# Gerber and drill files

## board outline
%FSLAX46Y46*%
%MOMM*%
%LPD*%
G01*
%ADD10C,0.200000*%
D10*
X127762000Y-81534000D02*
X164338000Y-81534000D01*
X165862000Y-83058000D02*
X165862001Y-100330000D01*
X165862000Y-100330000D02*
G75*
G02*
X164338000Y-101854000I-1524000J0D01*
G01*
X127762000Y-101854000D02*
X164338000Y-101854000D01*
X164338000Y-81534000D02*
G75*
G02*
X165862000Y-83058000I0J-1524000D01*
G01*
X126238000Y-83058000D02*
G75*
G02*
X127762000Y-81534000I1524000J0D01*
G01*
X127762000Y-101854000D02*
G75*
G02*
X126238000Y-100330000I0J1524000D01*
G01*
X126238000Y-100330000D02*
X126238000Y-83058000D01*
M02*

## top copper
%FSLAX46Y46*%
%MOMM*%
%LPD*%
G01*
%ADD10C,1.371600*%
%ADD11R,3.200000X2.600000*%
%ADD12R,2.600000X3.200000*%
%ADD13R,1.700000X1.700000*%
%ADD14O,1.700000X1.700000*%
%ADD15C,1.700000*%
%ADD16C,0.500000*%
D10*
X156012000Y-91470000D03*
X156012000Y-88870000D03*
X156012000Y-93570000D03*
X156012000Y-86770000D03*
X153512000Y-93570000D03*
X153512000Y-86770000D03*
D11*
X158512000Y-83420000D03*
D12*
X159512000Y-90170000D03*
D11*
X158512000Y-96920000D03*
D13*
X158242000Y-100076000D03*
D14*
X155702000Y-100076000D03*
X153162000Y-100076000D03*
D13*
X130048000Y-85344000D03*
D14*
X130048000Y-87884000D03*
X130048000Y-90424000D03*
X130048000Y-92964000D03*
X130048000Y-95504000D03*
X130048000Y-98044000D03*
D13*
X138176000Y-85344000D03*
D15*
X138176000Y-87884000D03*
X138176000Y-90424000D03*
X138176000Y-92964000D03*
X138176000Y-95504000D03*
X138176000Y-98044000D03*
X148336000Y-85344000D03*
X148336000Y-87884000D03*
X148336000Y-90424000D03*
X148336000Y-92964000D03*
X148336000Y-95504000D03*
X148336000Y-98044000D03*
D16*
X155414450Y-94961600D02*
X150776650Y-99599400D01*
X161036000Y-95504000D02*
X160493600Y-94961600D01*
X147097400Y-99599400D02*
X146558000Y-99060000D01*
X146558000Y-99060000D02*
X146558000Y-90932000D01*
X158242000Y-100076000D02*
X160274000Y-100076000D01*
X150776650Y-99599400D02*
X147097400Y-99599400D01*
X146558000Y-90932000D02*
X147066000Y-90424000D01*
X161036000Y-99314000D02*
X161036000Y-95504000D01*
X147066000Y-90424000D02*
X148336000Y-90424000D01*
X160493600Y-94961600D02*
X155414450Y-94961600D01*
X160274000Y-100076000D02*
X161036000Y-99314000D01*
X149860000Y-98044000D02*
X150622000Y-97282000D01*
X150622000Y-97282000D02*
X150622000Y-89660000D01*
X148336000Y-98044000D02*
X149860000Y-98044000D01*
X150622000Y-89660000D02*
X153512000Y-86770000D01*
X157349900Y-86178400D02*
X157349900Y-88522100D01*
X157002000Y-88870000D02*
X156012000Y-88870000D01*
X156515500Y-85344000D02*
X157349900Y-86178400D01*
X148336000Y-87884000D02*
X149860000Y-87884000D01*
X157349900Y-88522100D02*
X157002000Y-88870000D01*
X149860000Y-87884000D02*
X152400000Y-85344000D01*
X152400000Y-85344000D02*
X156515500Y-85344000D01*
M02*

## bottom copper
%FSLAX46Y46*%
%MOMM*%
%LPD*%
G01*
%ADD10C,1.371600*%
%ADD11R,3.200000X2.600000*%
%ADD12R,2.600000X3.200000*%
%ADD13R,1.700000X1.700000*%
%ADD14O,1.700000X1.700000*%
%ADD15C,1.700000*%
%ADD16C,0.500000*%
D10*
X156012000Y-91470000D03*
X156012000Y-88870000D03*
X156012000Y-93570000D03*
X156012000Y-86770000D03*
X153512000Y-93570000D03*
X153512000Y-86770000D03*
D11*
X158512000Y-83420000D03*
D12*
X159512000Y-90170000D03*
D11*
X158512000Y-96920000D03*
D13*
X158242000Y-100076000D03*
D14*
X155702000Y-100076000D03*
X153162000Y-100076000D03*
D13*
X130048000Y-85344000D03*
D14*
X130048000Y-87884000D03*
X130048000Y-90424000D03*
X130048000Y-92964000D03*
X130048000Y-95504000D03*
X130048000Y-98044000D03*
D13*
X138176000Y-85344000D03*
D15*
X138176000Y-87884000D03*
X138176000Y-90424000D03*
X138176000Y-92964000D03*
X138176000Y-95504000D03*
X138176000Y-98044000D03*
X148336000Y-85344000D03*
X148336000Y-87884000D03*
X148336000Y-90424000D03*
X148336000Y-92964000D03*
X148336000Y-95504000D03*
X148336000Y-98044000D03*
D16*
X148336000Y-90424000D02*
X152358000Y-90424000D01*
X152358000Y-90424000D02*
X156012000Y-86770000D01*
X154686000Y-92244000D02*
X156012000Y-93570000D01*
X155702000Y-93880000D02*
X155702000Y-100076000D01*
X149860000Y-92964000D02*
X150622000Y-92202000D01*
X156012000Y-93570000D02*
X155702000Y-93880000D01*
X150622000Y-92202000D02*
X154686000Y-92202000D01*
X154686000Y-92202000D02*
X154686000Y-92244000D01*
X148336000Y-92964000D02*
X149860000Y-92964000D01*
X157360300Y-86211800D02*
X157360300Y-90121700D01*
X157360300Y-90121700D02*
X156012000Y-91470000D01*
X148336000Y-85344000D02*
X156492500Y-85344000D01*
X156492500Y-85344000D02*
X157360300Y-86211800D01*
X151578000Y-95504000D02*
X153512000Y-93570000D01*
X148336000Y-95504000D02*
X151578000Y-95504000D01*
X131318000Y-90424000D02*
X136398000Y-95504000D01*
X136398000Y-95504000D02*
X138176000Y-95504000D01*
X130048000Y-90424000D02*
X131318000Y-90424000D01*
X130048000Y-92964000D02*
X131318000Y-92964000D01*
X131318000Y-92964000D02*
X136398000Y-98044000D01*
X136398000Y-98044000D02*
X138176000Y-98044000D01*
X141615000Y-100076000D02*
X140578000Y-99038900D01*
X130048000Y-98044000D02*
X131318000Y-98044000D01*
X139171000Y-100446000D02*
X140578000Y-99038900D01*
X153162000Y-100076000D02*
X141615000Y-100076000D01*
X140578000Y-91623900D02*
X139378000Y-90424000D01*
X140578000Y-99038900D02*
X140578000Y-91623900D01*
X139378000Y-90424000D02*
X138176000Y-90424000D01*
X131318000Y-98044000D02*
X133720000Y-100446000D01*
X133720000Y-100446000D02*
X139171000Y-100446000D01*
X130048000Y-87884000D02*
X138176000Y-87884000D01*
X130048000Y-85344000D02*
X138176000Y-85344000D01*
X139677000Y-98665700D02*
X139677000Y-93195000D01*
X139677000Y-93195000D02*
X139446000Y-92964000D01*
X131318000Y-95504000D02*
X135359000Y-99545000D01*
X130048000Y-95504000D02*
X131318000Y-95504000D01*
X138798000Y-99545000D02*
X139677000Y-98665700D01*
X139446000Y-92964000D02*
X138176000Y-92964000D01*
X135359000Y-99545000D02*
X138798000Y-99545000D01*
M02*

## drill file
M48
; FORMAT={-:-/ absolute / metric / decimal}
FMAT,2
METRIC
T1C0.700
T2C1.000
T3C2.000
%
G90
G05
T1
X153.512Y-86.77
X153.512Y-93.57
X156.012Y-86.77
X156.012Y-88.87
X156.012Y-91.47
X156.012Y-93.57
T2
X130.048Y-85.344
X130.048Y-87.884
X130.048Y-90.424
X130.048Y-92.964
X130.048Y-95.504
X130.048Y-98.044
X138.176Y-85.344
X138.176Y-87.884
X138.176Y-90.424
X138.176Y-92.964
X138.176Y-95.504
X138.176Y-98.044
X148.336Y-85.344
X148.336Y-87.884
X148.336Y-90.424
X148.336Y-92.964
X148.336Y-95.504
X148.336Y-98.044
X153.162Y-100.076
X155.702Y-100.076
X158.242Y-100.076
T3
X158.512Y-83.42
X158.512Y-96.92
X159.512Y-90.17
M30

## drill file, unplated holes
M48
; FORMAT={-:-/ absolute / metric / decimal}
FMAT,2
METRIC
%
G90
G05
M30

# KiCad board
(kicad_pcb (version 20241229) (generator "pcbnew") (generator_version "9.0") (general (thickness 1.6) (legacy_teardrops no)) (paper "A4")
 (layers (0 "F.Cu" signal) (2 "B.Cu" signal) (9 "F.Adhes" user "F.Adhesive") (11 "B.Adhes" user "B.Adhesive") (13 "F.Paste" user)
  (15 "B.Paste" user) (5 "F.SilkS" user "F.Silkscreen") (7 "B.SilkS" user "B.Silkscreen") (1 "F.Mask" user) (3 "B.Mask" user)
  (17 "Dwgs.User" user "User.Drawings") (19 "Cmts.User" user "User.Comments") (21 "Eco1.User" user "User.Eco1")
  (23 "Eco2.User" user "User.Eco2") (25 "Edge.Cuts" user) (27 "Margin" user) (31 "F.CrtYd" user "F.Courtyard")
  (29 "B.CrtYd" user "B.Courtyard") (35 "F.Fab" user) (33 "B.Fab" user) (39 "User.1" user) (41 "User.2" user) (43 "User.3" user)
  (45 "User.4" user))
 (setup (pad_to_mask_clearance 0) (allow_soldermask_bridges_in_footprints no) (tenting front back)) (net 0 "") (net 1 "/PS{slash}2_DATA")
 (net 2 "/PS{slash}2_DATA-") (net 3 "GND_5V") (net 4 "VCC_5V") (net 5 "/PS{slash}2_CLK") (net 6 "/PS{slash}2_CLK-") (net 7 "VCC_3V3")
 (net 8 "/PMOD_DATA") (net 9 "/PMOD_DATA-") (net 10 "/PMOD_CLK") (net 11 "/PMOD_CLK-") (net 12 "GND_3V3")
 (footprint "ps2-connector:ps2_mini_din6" (layer "F.Cu") (at 158.512 90.17 -90)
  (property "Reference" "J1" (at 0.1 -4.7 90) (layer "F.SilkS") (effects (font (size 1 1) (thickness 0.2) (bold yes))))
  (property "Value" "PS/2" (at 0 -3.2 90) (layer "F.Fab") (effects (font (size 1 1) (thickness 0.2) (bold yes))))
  (pad "1" thru_hole circle (at 1.3 2.5 90) (size 1.3716 1.3716) (drill 0.7) (layers "*.Cu" "*.Mask") (remove_unused_layers no)
   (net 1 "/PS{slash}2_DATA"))
  (pad "2" thru_hole circle (at -1.3 2.5 90) (size 1.3716 1.3716) (drill 0.7) (layers "*.Cu" "*.Mask") (remove_unused_layers no)
   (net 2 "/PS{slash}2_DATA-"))
  (pad "3" thru_hole circle (at 3.4 2.5 90) (size 1.3716 1.3716) (drill 0.7) (layers "*.Cu" "*.Mask") (remove_unused_layers no)
   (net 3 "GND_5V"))
  (pad "4" thru_hole circle (at -3.4 2.5 90) (size 1.3716 1.3716) (drill 0.7) (layers "*.Cu" "*.Mask") (remove_unused_layers no)
   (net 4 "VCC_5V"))
  (pad "5" thru_hole circle (at 3.4 5 90) (size 1.3716 1.3716) (drill 0.7) (layers "*.Cu" "*.Mask") (remove_unused_layers no)
   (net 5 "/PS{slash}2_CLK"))
  (pad "6" thru_hole circle (at -3.4 5 90) (size 1.3716 1.3716) (drill 0.7) (layers "*.Cu" "*.Mask") (remove_unused_layers no)
   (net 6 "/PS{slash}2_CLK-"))
  (pad "GND" thru_hole rect (at -6.75 0 90) (size 2.6 3.2) (drill 2) (layers "*.Cu" "*.Mask") (remove_unused_layers no)
   (thermal_bridge_angle 45))
  (pad "GND" thru_hole rect (at 0 -1 90) (size 3.2 2.6) (drill 2) (layers "*.Cu" "*.Mask") (remove_unused_layers no)
   (thermal_bridge_angle 45))
  (pad "GND" thru_hole rect (at 6.75 0 90) (size 2.6 3.2) (drill 2) (layers "*.Cu" "*.Mask") (remove_unused_layers no)
   (thermal_bridge_angle 45)))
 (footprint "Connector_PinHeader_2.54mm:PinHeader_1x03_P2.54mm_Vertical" (layer "F.Cu") (at 158.242 100.076 -90)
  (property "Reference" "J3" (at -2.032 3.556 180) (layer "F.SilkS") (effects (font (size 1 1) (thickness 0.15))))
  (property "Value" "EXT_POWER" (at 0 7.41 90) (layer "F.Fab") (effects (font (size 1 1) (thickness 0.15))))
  (pad "1" thru_hole rect (at 0 0 270) (size 1.7 1.7) (drill 1) (layers "*.Cu" "*.Mask") (remove_unused_layers no) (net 4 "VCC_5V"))
  (pad "2" thru_hole oval (at 0 2.54 270) (size 1.7 1.7) (drill 1) (layers "*.Cu" "*.Mask") (remove_unused_layers no) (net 3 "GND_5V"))
  (pad "3" thru_hole oval (at 0 5.08 270) (size 1.7 1.7) (drill 1) (layers "*.Cu" "*.Mask") (remove_unused_layers no) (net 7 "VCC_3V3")))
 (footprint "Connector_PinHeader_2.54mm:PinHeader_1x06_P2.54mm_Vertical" (layer "F.Cu") (at 130.048 85.344)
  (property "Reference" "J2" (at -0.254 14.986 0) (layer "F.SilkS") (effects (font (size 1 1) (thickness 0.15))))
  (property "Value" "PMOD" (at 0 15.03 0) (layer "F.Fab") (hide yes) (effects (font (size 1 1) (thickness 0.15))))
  (pad "1" thru_hole rect (at 0 0) (size 1.7 1.7) (drill 1) (layers "*.Cu" "*.Mask") (remove_unused_layers no) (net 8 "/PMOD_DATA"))
  (pad "2" thru_hole oval (at 0 2.54) (size 1.7 1.7) (drill 1) (layers "*.Cu" "*.Mask") (remove_unused_layers no) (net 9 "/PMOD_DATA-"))
  (pad "3" thru_hole oval (at 0 5.08) (size 1.7 1.7) (drill 1) (layers "*.Cu" "*.Mask") (remove_unused_layers no) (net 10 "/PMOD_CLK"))
  (pad "4" thru_hole oval (at 0 7.62) (size 1.7 1.7) (drill 1) (layers "*.Cu" "*.Mask") (remove_unused_layers no) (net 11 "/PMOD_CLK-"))
  (pad "5" thru_hole oval (at 0 10.16) (size 1.7 1.7) (drill 1) (layers "*.Cu" "*.Mask") (remove_unused_layers no) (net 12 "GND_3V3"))
  (pad "6" thru_hole oval (at 0 12.7) (size 1.7 1.7) (drill 1) (layers "*.Cu" "*.Mask") (remove_unused_layers no) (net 7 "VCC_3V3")))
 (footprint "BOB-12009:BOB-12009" (layer "F.Cu") (at 143.636 91.664)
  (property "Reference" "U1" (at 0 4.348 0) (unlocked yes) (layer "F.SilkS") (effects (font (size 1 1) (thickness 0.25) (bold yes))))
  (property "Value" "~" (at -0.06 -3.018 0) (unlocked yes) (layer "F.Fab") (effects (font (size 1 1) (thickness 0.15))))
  (pad "1" thru_hole rect (at -5.46 -6.32) (size 1.7 1.7) (drill 1) (layers "*.Cu" "*.Mask") (remove_unused_layers no) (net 8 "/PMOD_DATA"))
  (pad "2" thru_hole circle (at -5.46 -3.78) (size 1.7 1.7) (drill 1) (layers "*.Cu" "*.Mask") (remove_unused_layers no)
   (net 9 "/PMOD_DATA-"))
  (pad "3" thru_hole circle (at -5.46 -1.24) (size 1.7 1.7) (drill 1) (layers "*.Cu" "*.Mask") (remove_unused_layers no) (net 7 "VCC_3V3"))
  (pad "4" thru_hole circle (at -5.46 1.3) (size 1.7 1.7) (drill 1) (layers "*.Cu" "*.Mask") (remove_unused_layers no) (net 12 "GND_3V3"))
  (pad "5" thru_hole circle (at -5.46 3.84) (size 1.7 1.7) (drill 1) (layers "*.Cu" "*.Mask") (remove_unused_layers no) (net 10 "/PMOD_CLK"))
  (pad "6" thru_hole circle (at -5.46 6.38) (size 1.7 1.7) (drill 1) (layers "*.Cu" "*.Mask") (remove_unused_layers no)
   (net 11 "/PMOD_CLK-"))
  (pad "7" thru_hole circle (at 4.7 -6.32) (size 1.7 1.7) (drill 1) (layers "*.Cu" "*.Mask") (remove_unused_layers no)
   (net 1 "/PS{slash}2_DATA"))
  (pad "8" thru_hole circle (at 4.7 -3.78) (size 1.7 1.7) (drill 1) (layers "*.Cu" "*.Mask") (remove_unused_layers no)
   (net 2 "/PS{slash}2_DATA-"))
  (pad "9" thru_hole circle (at 4.7 -1.24) (size 1.7 1.7) (drill 1) (layers "*.Cu" "*.Mask") (remove_unused_layers no) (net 4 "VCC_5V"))
  (pad "10" thru_hole circle (at 4.7 1.3) (size 1.7 1.7) (drill 1) (layers "*.Cu" "*.Mask") (remove_unused_layers no) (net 3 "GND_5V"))
  (pad "11" thru_hole circle (at 4.7 3.84) (size 1.7 1.7) (drill 1) (layers "*.Cu" "*.Mask") (remove_unused_layers no)
   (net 5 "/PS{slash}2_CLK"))
  (pad "12" thru_hole circle (at 4.7 6.38) (size 1.7 1.7) (drill 1) (layers "*.Cu" "*.Mask") (remove_unused_layers no)
   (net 6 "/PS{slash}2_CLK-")))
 (gr_line (start 127.762 81.534) (end 164.338 81.534) (stroke (width 0.2) (type solid)) (layer "Edge.Cuts"))
 (gr_line (start 165.862 83.058) (end 165.862001 100.33) (stroke (width 0.2) (type solid)) (layer "Edge.Cuts"))
 (gr_arc (start 165.862 100.33) (mid 165.415631 101.407631) (end 164.338 101.854) (stroke (width 0.2) (type solid)) (layer "Edge.Cuts"))
 (gr_line (start 127.762 101.854) (end 164.338 101.854) (stroke (width 0.2) (type solid)) (layer "Edge.Cuts"))
 (gr_arc (start 164.338 81.534) (mid 165.415631 81.980369) (end 165.862 83.058) (stroke (width 0.2) (type solid)) (layer "Edge.Cuts"))
 (gr_arc (start 126.238 83.058) (mid 126.684369 81.980369) (end 127.762 81.534) (stroke (width 0.2) (type solid)) (layer "Edge.Cuts"))
 (gr_arc (start 127.762 101.854) (mid 126.684369 101.407631) (end 126.238 100.33) (stroke (width 0.2) (type solid)) (layer "Edge.Cuts"))
 (gr_line (start 126.238 100.33) (end 126.238 83.058) (stroke (width 0.2) (type solid)) (layer "Edge.Cuts"))
 (segment (start 155.41445 94.9616) (end 150.77665 99.5994) (width 0.5) (layer "F.Cu") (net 4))
 (segment (start 161.036 95.504) (end 160.4936 94.9616) (width 0.5) (layer "F.Cu") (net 4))
 (segment (start 147.0974 99.5994) (end 146.558 99.06) (width 0.5) (layer "F.Cu") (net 4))
 (segment (start 146.558 99.06) (end 146.558 90.932) (width 0.5) (layer "F.Cu") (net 4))
 (segment (start 158.242 100.076) (end 160.274 100.076) (width 0.5) (layer "F.Cu") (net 4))
 (segment (start 150.77665 99.5994) (end 147.0974 99.5994) (width 0.5) (layer "F.Cu") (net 4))
 (segment (start 146.558 90.932) (end 147.066 90.424) (width 0.5) (layer "F.Cu") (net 4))
 (segment (start 161.036 99.314) (end 161.036 95.504) (width 0.5) (layer "F.Cu") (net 4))
 (segment (start 147.066 90.424) (end 148.336 90.424) (width 0.5) (layer "F.Cu") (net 4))
 (segment (start 160.4936 94.9616) (end 155.41445 94.9616) (width 0.5) (layer "F.Cu") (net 4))
 (segment (start 160.274 100.076) (end 161.036 99.314) (width 0.5) (layer "F.Cu") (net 4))
 (segment (start 148.336 90.424) (end 152.358 90.424) (width 0.5) (layer "B.Cu") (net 4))
 (segment (start 152.358 90.424) (end 156.012 86.77) (width 0.5) (layer "B.Cu") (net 4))
 (segment (start 149.86 98.044) (end 150.622 97.282) (width 0.5) (layer "F.Cu") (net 6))
 (segment (start 150.622 97.282) (end 150.622 89.66) (width 0.5) (layer "F.Cu") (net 6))
 (segment (start 148.336 98.044) (end 149.86 98.044) (width 0.5) (layer "F.Cu") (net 6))
 (segment (start 150.622 89.66) (end 153.512 86.77) (width 0.5) (layer "F.Cu") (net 6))
 (segment (start 157.3499 86.1784) (end 157.3499 88.5221) (width 0.5) (layer "F.Cu") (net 2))
 (segment (start 157.002 88.87) (end 156.012 88.87) (width 0.5) (layer "F.Cu") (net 2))
 (segment (start 156.5155 85.344) (end 157.3499 86.1784) (width 0.5) (layer "F.Cu") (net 2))
 (segment (start 148.336 87.884) (end 149.86 87.884) (width 0.5) (layer "F.Cu") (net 2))
 (segment (start 157.3499 88.5221) (end 157.002 88.87) (width 0.5) (layer "F.Cu") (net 2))
 (segment (start 149.86 87.884) (end 152.4 85.344) (width 0.5) (layer "F.Cu") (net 2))
 (segment (start 152.4 85.344) (end 156.5155 85.344) (width 0.5) (layer "F.Cu") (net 2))
 (segment (start 154.686 92.244) (end 156.012 93.57) (width 0.5) (layer "B.Cu") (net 3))
 (segment (start 155.702 93.88) (end 155.702 100.076) (width 0.5) (layer "B.Cu") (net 3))
 (segment (start 149.86 92.964) (end 150.622 92.202) (width 0.5) (layer "B.Cu") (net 3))
 (segment (start 156.012 93.57) (end 155.702 93.88) (width 0.5) (layer "B.Cu") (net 3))
 (segment (start 150.622 92.202) (end 154.686 92.202) (width 0.5) (layer "B.Cu") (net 3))
 (segment (start 154.686 92.202) (end 154.686 92.244) (width 0.5) (layer "B.Cu") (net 3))
 (segment (start 148.336 92.964) (end 149.86 92.964) (width 0.5) (layer "B.Cu") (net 3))
 (segment (start 157.3603 86.2118) (end 157.3603 90.1217) (width 0.5) (layer "B.Cu") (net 1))
 (segment (start 157.3603 90.1217) (end 156.012 91.47) (width 0.5) (layer "B.Cu") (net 1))
 (segment (start 148.336 85.344) (end 156.4925 85.344) (width 0.5) (layer "B.Cu") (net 1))
 (segment (start 156.4925 85.344) (end 157.3603 86.2118) (width 0.5) (layer "B.Cu") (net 1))
 (segment (start 151.578 95.504) (end 153.512 93.57) (width 0.5) (layer "B.Cu") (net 5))
 (segment (start 148.336 95.504) (end 151.578 95.504) (width 0.5) (layer "B.Cu") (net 5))
 (segment (start 131.318 90.424) (end 136.398 95.504) (width 0.5) (layer "B.Cu") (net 10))
 (segment (start 136.398 95.504) (end 138.176 95.504) (width 0.5) (layer "B.Cu") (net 10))
 (segment (start 130.048 90.424) (end 131.318 90.424) (width 0.5) (layer "B.Cu") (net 10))
 (segment (start 130.048 92.964) (end 131.318 92.964) (width 0.5) (layer "B.Cu") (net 11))
 (segment (start 131.318 92.964) (end 136.398 98.044) (width 0.5) (layer "B.Cu") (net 11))
 (segment (start 136.398 98.044) (end 138.176 98.044) (width 0.5) (layer "B.Cu") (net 11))
 (segment (start 141.615 100.076) (end 140.578 99.0389) (width 0.5) (layer "B.Cu") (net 7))
 (segment (start 130.048 98.044) (end 131.318 98.044) (width 0.5) (layer "B.Cu") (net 7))
 (segment (start 139.171 100.446) (end 140.578 99.0389) (width 0.5) (layer "B.Cu") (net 7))
 (segment (start 153.162 100.076) (end 141.615 100.076) (width 0.5) (layer "B.Cu") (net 7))
 (segment (start 140.578 91.6239) (end 139.378 90.424) (width 0.5) (layer "B.Cu") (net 7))
 (segment (start 140.578 99.0389) (end 140.578 91.6239) (width 0.5) (layer "B.Cu") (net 7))
 (segment (start 139.378 90.424) (end 138.176 90.424) (width 0.5) (layer "B.Cu") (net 7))
 (segment (start 131.318 98.044) (end 133.72 100.446) (width 0.5) (layer "B.Cu") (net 7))
 (segment (start 133.72 100.446) (end 139.171 100.446) (width 0.5) (layer "B.Cu") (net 7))
 (segment (start 130.048 87.884) (end 138.176 87.884) (width 0.5) (layer "B.Cu") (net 9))
 (segment (start 130.048 85.344) (end 138.176 85.344) (width 0.5) (layer "B.Cu") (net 8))
 (segment (start 139.677 98.6657) (end 139.677 93.195) (width 0.5) (layer "B.Cu") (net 12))
 (segment (start 139.677 93.195) (end 139.446 92.964) (width 0.5) (layer "B.Cu") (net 12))
 (segment (start 131.318 95.504) (end 135.359 99.545) (width 0.5) (layer "B.Cu") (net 12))
 (segment (start 130.048 95.504) (end 131.318 95.504) (width 0.5) (layer "B.Cu") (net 12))
 (segment (start 138.798 99.545) (end 139.677 98.6657) (width 0.5) (layer "B.Cu") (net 12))
 (segment (start 139.446 92.964) (end 138.176 92.964) (width 0.5) (layer "B.Cu") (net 12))
 (segment (start 135.359 99.545) (end 138.798 99.545) (width 0.5) (layer "B.Cu") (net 12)))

